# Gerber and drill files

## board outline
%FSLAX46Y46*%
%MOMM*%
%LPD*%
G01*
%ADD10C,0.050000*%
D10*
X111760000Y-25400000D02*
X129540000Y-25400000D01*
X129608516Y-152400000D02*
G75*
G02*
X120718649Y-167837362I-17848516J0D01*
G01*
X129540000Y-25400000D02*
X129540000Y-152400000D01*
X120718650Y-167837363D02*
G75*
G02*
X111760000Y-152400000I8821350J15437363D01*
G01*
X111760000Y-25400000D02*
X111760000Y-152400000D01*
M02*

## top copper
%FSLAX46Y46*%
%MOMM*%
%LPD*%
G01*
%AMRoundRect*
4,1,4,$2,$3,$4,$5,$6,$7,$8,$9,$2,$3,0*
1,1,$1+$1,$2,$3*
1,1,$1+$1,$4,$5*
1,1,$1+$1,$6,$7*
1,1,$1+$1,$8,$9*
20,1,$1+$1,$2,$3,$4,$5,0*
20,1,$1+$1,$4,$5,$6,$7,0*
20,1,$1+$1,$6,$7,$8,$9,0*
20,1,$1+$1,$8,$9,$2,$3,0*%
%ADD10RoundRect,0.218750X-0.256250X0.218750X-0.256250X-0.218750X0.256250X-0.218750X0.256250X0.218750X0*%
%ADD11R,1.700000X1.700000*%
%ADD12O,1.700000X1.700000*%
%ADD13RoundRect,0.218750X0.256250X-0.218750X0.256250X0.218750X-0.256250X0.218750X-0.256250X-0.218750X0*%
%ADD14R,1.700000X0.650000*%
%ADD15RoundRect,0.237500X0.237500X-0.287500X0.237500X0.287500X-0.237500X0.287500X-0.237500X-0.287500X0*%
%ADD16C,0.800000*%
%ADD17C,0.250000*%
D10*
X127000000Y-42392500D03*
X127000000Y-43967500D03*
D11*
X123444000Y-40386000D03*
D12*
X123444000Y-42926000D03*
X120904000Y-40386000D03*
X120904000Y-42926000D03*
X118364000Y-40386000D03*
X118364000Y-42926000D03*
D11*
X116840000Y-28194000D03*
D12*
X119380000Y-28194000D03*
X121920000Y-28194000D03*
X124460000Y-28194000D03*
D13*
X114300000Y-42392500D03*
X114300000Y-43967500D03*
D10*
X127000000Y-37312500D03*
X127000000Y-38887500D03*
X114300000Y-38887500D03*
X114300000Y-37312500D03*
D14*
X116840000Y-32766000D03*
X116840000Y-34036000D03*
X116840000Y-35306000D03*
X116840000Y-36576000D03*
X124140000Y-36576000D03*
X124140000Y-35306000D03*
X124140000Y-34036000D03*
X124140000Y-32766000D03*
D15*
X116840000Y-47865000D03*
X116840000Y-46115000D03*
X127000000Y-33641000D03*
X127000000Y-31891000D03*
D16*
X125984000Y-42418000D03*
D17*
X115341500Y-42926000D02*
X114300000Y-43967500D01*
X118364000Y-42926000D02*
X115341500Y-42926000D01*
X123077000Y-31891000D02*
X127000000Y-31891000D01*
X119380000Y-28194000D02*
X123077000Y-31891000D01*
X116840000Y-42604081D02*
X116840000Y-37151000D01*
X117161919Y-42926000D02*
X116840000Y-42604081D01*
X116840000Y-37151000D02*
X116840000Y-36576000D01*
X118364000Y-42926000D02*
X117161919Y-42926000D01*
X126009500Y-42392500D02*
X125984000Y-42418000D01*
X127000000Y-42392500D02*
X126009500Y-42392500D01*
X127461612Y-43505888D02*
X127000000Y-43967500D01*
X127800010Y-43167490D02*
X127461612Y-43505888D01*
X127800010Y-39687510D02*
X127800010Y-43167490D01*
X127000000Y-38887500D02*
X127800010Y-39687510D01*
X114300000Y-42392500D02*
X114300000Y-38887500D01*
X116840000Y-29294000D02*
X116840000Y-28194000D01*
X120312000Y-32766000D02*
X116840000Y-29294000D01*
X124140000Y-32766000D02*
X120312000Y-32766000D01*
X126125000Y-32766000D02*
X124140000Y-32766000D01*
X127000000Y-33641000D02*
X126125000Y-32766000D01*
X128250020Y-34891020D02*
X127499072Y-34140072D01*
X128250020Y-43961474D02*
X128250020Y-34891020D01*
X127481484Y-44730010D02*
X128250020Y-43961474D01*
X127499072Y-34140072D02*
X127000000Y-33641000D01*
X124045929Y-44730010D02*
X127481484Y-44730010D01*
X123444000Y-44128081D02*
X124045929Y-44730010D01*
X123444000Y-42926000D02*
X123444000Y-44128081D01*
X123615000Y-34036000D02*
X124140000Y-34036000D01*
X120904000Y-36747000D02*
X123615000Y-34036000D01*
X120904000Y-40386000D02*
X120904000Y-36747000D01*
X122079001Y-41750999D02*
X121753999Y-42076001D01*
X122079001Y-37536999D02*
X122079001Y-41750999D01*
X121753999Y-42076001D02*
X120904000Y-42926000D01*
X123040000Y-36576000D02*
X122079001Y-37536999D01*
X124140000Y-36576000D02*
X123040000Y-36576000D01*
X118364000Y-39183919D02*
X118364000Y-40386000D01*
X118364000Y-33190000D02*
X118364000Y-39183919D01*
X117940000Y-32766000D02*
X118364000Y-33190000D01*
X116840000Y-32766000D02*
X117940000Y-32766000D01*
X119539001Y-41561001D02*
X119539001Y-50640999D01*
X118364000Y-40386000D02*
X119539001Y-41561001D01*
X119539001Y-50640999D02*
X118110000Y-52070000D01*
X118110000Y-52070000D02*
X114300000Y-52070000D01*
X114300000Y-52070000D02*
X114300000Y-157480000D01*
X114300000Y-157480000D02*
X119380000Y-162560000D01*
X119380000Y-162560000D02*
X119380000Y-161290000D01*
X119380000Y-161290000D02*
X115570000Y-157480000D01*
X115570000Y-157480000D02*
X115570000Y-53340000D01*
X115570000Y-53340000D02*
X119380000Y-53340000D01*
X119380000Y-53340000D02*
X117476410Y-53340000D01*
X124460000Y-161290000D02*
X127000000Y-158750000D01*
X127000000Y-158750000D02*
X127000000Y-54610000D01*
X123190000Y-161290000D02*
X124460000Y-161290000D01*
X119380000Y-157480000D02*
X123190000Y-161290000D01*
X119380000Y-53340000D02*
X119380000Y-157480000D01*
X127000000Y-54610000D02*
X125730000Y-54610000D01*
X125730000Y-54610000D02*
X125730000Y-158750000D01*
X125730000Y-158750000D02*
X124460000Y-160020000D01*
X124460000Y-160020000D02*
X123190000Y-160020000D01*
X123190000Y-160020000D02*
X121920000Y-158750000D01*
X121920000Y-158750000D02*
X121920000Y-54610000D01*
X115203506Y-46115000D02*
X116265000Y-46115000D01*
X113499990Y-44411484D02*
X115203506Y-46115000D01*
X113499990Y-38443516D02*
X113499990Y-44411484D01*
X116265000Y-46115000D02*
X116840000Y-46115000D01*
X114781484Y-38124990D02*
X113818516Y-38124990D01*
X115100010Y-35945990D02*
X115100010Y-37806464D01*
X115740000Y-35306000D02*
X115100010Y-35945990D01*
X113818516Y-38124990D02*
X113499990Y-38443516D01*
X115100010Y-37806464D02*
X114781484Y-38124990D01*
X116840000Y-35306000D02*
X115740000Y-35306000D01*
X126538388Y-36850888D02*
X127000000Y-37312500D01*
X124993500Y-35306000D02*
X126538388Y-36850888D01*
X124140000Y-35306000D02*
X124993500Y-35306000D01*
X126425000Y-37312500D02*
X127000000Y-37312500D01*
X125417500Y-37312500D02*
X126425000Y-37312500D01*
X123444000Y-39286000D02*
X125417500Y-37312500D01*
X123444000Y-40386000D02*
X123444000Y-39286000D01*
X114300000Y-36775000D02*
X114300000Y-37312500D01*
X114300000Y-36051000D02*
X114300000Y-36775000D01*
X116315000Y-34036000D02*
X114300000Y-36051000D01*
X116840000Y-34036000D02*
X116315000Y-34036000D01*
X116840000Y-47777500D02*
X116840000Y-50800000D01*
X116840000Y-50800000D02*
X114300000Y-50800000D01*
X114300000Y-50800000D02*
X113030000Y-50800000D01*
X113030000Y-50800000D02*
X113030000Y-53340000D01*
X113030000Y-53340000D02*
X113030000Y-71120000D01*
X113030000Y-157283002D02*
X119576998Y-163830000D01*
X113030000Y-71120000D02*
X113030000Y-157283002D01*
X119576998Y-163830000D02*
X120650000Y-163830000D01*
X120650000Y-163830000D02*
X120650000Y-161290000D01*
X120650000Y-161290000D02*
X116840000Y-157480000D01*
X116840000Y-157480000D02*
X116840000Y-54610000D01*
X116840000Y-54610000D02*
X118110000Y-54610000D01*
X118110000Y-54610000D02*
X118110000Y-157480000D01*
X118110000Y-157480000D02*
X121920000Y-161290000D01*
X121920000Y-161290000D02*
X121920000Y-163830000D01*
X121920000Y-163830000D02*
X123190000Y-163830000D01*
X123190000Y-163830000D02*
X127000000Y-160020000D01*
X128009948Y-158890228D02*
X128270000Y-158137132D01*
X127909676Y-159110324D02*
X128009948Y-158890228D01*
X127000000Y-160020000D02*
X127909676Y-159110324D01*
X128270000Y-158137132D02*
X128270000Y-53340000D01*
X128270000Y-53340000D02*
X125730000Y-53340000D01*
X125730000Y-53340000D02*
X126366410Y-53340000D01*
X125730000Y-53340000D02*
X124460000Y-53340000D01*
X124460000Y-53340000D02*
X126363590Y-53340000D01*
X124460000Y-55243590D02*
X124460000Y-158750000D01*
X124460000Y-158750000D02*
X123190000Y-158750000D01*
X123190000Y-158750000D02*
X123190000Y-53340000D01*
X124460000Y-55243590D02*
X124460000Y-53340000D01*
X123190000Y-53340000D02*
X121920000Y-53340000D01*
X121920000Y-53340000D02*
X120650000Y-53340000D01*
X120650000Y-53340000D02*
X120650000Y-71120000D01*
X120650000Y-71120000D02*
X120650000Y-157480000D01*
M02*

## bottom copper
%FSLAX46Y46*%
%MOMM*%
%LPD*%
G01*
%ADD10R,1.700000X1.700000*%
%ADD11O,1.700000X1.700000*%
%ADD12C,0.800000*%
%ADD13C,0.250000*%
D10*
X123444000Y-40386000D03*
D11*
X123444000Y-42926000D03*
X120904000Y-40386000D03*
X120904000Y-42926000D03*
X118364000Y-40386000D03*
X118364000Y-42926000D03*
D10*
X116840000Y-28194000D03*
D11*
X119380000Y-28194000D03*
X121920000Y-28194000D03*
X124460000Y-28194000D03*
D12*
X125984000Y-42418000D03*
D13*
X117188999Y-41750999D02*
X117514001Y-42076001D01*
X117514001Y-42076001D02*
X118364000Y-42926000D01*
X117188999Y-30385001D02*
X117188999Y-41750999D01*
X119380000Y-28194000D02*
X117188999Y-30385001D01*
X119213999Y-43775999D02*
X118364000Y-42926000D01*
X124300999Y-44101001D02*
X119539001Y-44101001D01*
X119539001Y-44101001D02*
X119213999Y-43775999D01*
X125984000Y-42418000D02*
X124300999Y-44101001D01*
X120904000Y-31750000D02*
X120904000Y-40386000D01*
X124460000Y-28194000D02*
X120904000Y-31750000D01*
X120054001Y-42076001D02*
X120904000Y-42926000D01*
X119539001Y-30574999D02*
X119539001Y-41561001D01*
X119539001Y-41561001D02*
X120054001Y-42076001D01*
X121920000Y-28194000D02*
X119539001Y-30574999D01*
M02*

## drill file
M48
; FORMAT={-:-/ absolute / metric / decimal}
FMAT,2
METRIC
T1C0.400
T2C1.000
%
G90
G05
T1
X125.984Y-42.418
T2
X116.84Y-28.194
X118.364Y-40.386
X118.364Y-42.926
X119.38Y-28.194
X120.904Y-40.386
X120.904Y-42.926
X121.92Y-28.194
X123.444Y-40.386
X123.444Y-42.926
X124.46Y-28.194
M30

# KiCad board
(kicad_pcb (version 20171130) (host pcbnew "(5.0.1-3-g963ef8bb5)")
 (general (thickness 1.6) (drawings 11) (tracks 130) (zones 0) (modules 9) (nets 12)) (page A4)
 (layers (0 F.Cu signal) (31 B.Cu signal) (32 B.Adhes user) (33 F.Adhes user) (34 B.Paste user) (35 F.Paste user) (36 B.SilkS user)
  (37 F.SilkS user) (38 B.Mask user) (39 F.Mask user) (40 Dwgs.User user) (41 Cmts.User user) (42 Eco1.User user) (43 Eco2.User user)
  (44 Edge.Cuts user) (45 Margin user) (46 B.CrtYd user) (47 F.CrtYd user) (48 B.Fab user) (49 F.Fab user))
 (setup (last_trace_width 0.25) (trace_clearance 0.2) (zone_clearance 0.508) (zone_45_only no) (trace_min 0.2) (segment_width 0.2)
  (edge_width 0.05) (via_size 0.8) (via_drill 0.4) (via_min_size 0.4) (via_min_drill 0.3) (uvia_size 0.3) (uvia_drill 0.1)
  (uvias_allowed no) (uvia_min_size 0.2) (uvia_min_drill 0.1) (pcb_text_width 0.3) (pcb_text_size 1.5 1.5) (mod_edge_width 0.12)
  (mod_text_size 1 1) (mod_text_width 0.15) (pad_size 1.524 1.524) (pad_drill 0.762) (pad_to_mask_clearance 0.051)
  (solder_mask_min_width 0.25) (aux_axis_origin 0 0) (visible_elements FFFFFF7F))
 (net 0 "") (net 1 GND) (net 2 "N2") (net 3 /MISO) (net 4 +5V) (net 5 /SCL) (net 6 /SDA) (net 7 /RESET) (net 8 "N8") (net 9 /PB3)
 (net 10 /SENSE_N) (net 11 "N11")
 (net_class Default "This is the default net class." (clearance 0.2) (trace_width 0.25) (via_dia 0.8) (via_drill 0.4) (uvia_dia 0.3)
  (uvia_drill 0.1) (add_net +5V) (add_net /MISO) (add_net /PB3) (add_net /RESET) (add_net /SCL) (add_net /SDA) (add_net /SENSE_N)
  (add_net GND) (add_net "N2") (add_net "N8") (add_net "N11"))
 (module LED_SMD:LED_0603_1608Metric (layer F.Cu) (at 127 43.18 270)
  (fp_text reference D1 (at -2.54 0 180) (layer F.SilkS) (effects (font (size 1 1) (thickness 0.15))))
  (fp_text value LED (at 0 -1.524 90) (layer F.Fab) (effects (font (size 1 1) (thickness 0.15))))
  (pad 1 smd roundrect (at -0.7875 0 270) (size 0.875 0.95) (layers F.Cu F.Paste F.Mask) (roundrect_rratio 0.25) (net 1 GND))
  (pad 2 smd roundrect (at 0.7875 0 270) (size 0.875 0.95) (layers F.Cu F.Paste F.Mask) (roundrect_rratio 0.25) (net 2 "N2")))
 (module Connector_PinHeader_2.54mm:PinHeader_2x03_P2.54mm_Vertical (layer F.Cu) (at 123.444 40.386 270)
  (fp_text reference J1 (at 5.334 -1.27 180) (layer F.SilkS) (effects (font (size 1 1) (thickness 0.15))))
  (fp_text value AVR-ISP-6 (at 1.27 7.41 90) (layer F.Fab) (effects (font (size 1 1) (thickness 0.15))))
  (pad 1 thru_hole rect (at 0 0 270) (size 1.7 1.7) (drill 1) (layers *.Cu *.Mask) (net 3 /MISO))
  (pad 2 thru_hole oval (at 2.54 0 270) (size 1.7 1.7) (drill 1) (layers *.Cu *.Mask) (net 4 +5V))
  (pad 3 thru_hole oval (at 0 2.54 270) (size 1.7 1.7) (drill 1) (layers *.Cu *.Mask) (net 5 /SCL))
  (pad 4 thru_hole oval (at 2.54 2.54 270) (size 1.7 1.7) (drill 1) (layers *.Cu *.Mask) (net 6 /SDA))
  (pad 5 thru_hole oval (at 0 5.08 270) (size 1.7 1.7) (drill 1) (layers *.Cu *.Mask) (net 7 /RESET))
  (pad 6 thru_hole oval (at 2.54 5.08 270) (size 1.7 1.7) (drill 1) (layers *.Cu *.Mask) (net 1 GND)))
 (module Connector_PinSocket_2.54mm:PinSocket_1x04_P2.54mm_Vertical (layer F.Cu) (at 116.84 28.194 90)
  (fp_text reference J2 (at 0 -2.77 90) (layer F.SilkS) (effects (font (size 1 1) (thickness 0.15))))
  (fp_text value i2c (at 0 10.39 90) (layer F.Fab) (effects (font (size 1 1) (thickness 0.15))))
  (pad 1 thru_hole rect (at 0 0 90) (size 1.7 1.7) (drill 1) (layers *.Cu *.Mask) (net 4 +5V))
  (pad 2 thru_hole oval (at 0 2.54 90) (size 1.7 1.7) (drill 1) (layers *.Cu *.Mask) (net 1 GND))
  (pad 3 thru_hole oval (at 0 5.08 90) (size 1.7 1.7) (drill 1) (layers *.Cu *.Mask) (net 6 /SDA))
  (pad 4 thru_hole oval (at 0 7.62 90) (size 1.7 1.7) (drill 1) (layers *.Cu *.Mask) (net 5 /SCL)))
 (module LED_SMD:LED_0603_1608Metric (layer F.Cu) (at 114.3 43.18 90)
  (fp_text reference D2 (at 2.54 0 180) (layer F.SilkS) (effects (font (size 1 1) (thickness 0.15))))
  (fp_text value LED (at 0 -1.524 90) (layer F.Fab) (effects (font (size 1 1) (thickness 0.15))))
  (pad 2 smd roundrect (at 0.7875 0 90) (size 0.875 0.95) (layers F.Cu F.Paste F.Mask) (roundrect_rratio 0.25) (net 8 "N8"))
  (pad 1 smd roundrect (at -0.7875 0 90) (size 0.875 0.95) (layers F.Cu F.Paste F.Mask) (roundrect_rratio 0.25) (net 1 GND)))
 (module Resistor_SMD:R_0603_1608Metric (layer F.Cu) (at 127 38.1 270)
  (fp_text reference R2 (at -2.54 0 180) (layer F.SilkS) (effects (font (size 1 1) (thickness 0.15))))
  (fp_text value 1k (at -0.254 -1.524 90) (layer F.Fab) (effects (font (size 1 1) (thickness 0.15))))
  (pad 1 smd roundrect (at -0.7875 0 270) (size 0.875 0.95) (layers F.Cu F.Paste F.Mask) (roundrect_rratio 0.25) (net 3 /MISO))
  (pad 2 smd roundrect (at 0.7875 0 270) (size 0.875 0.95) (layers F.Cu F.Paste F.Mask) (roundrect_rratio 0.25) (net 2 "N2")))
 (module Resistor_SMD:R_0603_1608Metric (layer F.Cu) (at 114.3 38.1 270)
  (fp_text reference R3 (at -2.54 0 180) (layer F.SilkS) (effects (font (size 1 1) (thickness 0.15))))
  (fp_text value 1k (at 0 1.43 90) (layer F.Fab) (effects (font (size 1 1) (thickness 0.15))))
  (pad 2 smd roundrect (at 0.7875 0 270) (size 0.875 0.95) (layers F.Cu F.Paste F.Mask) (roundrect_rratio 0.25) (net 8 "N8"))
  (pad 1 smd roundrect (at -0.7875 0 270) (size 0.875 0.95) (layers F.Cu F.Paste F.Mask) (roundrect_rratio 0.25) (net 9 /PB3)))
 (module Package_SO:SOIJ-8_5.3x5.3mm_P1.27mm (layer F.Cu) (at 120.49 34.671)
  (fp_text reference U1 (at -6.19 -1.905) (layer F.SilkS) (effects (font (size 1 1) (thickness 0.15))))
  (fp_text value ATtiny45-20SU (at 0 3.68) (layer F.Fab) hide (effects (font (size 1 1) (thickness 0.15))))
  (pad 1 smd rect (at -3.65 -1.905) (size 1.7 0.65) (layers F.Cu F.Paste F.Mask) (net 7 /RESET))
  (pad 2 smd rect (at -3.65 -0.635) (size 1.7 0.65) (layers F.Cu F.Paste F.Mask) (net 9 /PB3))
  (pad 3 smd rect (at -3.65 0.635) (size 1.7 0.65) (layers F.Cu F.Paste F.Mask) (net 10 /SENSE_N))
  (pad 4 smd rect (at -3.65 1.905) (size 1.7 0.65) (layers F.Cu F.Paste F.Mask) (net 1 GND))
  (pad 5 smd rect (at 3.65 1.905) (size 1.7 0.65) (layers F.Cu F.Paste F.Mask) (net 6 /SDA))
  (pad 6 smd rect (at 3.65 0.635) (size 1.7 0.65) (layers F.Cu F.Paste F.Mask) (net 3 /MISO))
  (pad 7 smd rect (at 3.65 -0.635) (size 1.7 0.65) (layers F.Cu F.Paste F.Mask) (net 5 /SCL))
  (pad 8 smd rect (at 3.65 -1.905) (size 1.7 0.65) (layers F.Cu F.Paste F.Mask) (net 4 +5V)))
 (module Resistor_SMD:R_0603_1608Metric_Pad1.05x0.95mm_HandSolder (layer F.Cu) (at 116.84 46.99 90)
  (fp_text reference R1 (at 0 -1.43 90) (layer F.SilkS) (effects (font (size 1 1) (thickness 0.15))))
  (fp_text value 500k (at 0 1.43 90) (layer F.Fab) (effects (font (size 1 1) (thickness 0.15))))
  (pad 1 smd roundrect (at -0.875 0 90) (size 1.05 0.95) (layers F.Cu F.Paste F.Mask) (roundrect_rratio 0.25) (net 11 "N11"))
  (pad 2 smd roundrect (at 0.875 0 90) (size 1.05 0.95) (layers F.Cu F.Paste F.Mask) (roundrect_rratio 0.25) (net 10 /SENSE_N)))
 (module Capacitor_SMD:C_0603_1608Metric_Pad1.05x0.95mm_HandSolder (layer F.Cu) (at 127 32.766 90)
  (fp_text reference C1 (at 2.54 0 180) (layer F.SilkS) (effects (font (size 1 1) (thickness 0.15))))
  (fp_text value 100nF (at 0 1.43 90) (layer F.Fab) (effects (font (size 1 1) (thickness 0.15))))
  (pad 1 smd roundrect (at -0.875 0 90) (size 1.05 0.95) (layers F.Cu F.Paste F.Mask) (roundrect_rratio 0.25) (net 4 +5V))
  (pad 2 smd roundrect (at 0.875 0 90) (size 1.05 0.95) (layers F.Cu F.Paste F.Mask) (roundrect_rratio 0.25) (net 1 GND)))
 (gr_line (start 111.76 25.4) (end 129.54 25.4) (layer Edge.Cuts) (width 0.05))
 (gr_arc (start 111.76 152.4) (end 120.718649 167.837362) (angle -59.87243964) (layer Edge.Cuts) (width 0.05))
 (gr_line (start 129.54 25.4) (end 129.54 152.4) (layer Edge.Cuts) (width 0.05))
 (gr_arc (start 129.54 152.4) (end 111.76 152.4) (angle -60.2551187) (layer Edge.Cuts) (width 0.05))
 (gr_line (start 111.76 25.4) (end 111.76 152.4) (layer Edge.Cuts) (width 0.05))
 (segment (start 115.3415 42.926) (end 114.3 43.9675) (width 0.25) (layer F.Cu) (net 1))
 (segment (start 118.364 42.926) (end 115.3415 42.926) (width 0.25) (layer F.Cu) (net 1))
 (segment (start 123.077 31.891) (end 127 31.891) (width 0.25) (layer F.Cu) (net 1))
 (segment (start 119.38 28.194) (end 123.077 31.891) (width 0.25) (layer F.Cu) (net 1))
 (segment (start 116.84 42.604081) (end 116.84 37.151) (width 0.25) (layer F.Cu) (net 1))
 (segment (start 117.161919 42.926) (end 116.84 42.604081) (width 0.25) (layer F.Cu) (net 1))
 (segment (start 116.84 37.151) (end 116.84 36.576) (width 0.25) (layer F.Cu) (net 1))
 (segment (start 118.364 42.926) (end 117.161919 42.926) (width 0.25) (layer F.Cu) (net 1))
 (segment (start 117.188999 41.750999) (end 117.514001 42.076001) (width 0.25) (layer B.Cu) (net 1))
 (segment (start 117.514001 42.076001) (end 118.364 42.926) (width 0.25) (layer B.Cu) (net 1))
 (segment (start 117.188999 30.385001) (end 117.188999 41.750999) (width 0.25) (layer B.Cu) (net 1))
 (segment (start 119.38 28.194) (end 117.188999 30.385001) (width 0.25) (layer B.Cu) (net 1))
 (via (at 125.984 42.418) (size 0.8) (drill 0.4) (layers F.Cu B.Cu) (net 1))
 (segment (start 126.0095 42.3925) (end 125.984 42.418) (width 0.25) (layer F.Cu) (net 1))
 (segment (start 127 42.3925) (end 126.0095 42.3925) (width 0.25) (layer F.Cu) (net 1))
 (segment (start 119.213999 43.775999) (end 118.364 42.926) (width 0.25) (layer B.Cu) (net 1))
 (segment (start 124.300999 44.101001) (end 119.539001 44.101001) (width 0.25) (layer B.Cu) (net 1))
 (segment (start 119.539001 44.101001) (end 119.213999 43.775999) (width 0.25) (layer B.Cu) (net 1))
 (segment (start 125.984 42.418) (end 124.300999 44.101001) (width 0.25) (layer B.Cu) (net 1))
 (segment (start 127.461612 43.505888) (end 127 43.9675) (width 0.25) (layer F.Cu) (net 2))
 (segment (start 127.80001 43.16749) (end 127.461612 43.505888) (width 0.25) (layer F.Cu) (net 2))
 (segment (start 127.80001 39.68751) (end 127.80001 43.16749) (width 0.25) (layer F.Cu) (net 2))
 (segment (start 127 38.8875) (end 127.80001 39.68751) (width 0.25) (layer F.Cu) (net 2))
 (segment (start 114.3 42.3925) (end 114.3 38.8875) (width 0.25) (layer F.Cu) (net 8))
 (segment (start 116.84 29.294) (end 116.84 28.194) (width 0.25) (layer F.Cu) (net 4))
 (segment (start 120.312 32.766) (end 116.84 29.294) (width 0.25) (layer F.Cu) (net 4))
 (segment (start 124.14 32.766) (end 120.312 32.766) (width 0.25) (layer F.Cu) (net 4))
 (segment (start 126.125 32.766) (end 124.14 32.766) (width 0.25) (layer F.Cu) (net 4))
 (segment (start 127 33.641) (end 126.125 32.766) (width 0.25) (layer F.Cu) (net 4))
 (segment (start 128.25002 34.89102) (end 127.499072 34.140072) (width 0.25) (layer F.Cu) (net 4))
 (segment (start 128.25002 43.961474) (end 128.25002 34.89102) (width 0.25) (layer F.Cu) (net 4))
 (segment (start 127.481484 44.73001) (end 128.25002 43.961474) (width 0.25) (layer F.Cu) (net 4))
 (segment (start 127.499072 34.140072) (end 127 33.641) (width 0.25) (layer F.Cu) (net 4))
 (segment (start 124.045929 44.73001) (end 127.481484 44.73001) (width 0.25) (layer F.Cu) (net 4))
 (segment (start 123.444 44.128081) (end 124.045929 44.73001) (width 0.25) (layer F.Cu) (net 4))
 (segment (start 123.444 42.926) (end 123.444 44.128081) (width 0.25) (layer F.Cu) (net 4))
 (segment (start 123.615 34.036) (end 124.14 34.036) (width 0.25) (layer F.Cu) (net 5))
 (segment (start 120.904 36.747) (end 123.615 34.036) (width 0.25) (layer F.Cu) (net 5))
 (segment (start 120.904 40.386) (end 120.904 36.747) (width 0.25) (layer F.Cu) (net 5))
 (segment (start 120.904 31.75) (end 120.904 40.386) (width 0.25) (layer B.Cu) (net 5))
 (segment (start 124.46 28.194) (end 120.904 31.75) (width 0.25) (layer B.Cu) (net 5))
 (segment (start 120.054001 42.076001) (end 120.904 42.926) (width 0.25) (layer B.Cu) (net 6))
 (segment (start 119.539001 30.574999) (end 119.539001 41.561001) (width 0.25) (layer B.Cu) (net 6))
 (segment (start 119.539001 41.561001) (end 120.054001 42.076001) (width 0.25) (layer B.Cu) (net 6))
 (segment (start 121.92 28.194) (end 119.539001 30.574999) (width 0.25) (layer B.Cu) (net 6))
 (segment (start 122.079001 41.750999) (end 121.753999 42.076001) (width 0.25) (layer F.Cu) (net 6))
 (segment (start 122.079001 37.536999) (end 122.079001 41.750999) (width 0.25) (layer F.Cu) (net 6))
 (segment (start 121.753999 42.076001) (end 120.904 42.926) (width 0.25) (layer F.Cu) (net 6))
 (segment (start 123.04 36.576) (end 122.079001 37.536999) (width 0.25) (layer F.Cu) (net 6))
 (segment (start 124.14 36.576) (end 123.04 36.576) (width 0.25) (layer F.Cu) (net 6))
 (segment (start 118.364 39.183919) (end 118.364 40.386) (width 0.25) (layer F.Cu) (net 7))
 (segment (start 118.364 33.19) (end 118.364 39.183919) (width 0.25) (layer F.Cu) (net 7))
 (segment (start 117.94 32.766) (end 118.364 33.19) (width 0.25) (layer F.Cu) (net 7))
 (segment (start 116.84 32.766) (end 117.94 32.766) (width 0.25) (layer F.Cu) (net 7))
 (segment (start 119.539001 41.561001) (end 119.539001 50.640999) (width 0.25) (layer F.Cu) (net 7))
 (segment (start 118.364 40.386) (end 119.539001 41.561001) (width 0.25) (layer F.Cu) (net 7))
 (segment (start 119.539001 50.640999) (end 118.11 52.07) (width 0.25) (layer F.Cu) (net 7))
 (segment (start 118.11 52.07) (end 114.3 52.07) (width 0.25) (layer F.Cu) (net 7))
 (segment (start 114.3 52.07) (end 114.3 157.48) (width 0.25) (layer F.Cu) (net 7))
 (segment (start 114.3 157.48) (end 119.38 162.56) (width 0.25) (layer F.Cu) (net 7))
 (segment (start 119.38 162.56) (end 119.38 161.29) (width 0.25) (layer F.Cu) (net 7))
 (segment (start 119.38 161.29) (end 115.57 157.48) (width 0.25) (layer F.Cu) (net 7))
 (segment (start 115.57 157.48) (end 115.57 53.34) (width 0.25) (layer F.Cu) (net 7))
 (segment (start 115.57 53.34) (end 119.38 53.34) (width 0.25) (layer F.Cu) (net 7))
 (segment (start 119.38 53.34) (end 117.47641 53.34) (width 0.25) (layer F.Cu) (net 7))
 (segment (start 124.46 161.29) (end 127 158.75) (width 0.25) (layer F.Cu) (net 7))
 (segment (start 127 158.75) (end 127 54.61) (width 0.25) (layer F.Cu) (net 7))
 (segment (start 123.19 161.29) (end 124.46 161.29) (width 0.25) (layer F.Cu) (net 7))
 (segment (start 119.38 157.48) (end 123.19 161.29) (width 0.25) (layer F.Cu) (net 7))
 (segment (start 119.38 53.34) (end 119.38 157.48) (width 0.25) (layer F.Cu) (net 7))
 (segment (start 127 54.61) (end 125.73 54.61) (width 0.25) (layer F.Cu) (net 7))
 (segment (start 125.73 54.61) (end 125.73 158.75) (width 0.25) (layer F.Cu) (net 7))
 (segment (start 125.73 158.75) (end 124.46 160.02) (width 0.25) (layer F.Cu) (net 7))
 (segment (start 124.46 160.02) (end 123.19 160.02) (width 0.25) (layer F.Cu) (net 7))
 (segment (start 123.19 160.02) (end 121.92 158.75) (width 0.25) (layer F.Cu) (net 7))
 (segment (start 121.92 158.75) (end 121.92 54.61) (width 0.25) (layer F.Cu) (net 7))
 (segment (start 115.203506 46.115) (end 116.265 46.115) (width 0.25) (layer F.Cu) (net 10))
 (segment (start 113.49999 44.411484) (end 115.203506 46.115) (width 0.25) (layer F.Cu) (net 10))
 (segment (start 113.49999 38.443516) (end 113.49999 44.411484) (width 0.25) (layer F.Cu) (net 10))
 (segment (start 116.265 46.115) (end 116.84 46.115) (width 0.25) (layer F.Cu) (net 10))
 (segment (start 114.781484 38.12499) (end 113.818516 38.12499) (width 0.25) (layer F.Cu) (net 10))
 (segment (start 115.10001 35.94599) (end 115.10001 37.806464) (width 0.25) (layer F.Cu) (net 10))
 (segment (start 115.74 35.306) (end 115.10001 35.94599) (width 0.25) (layer F.Cu) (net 10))
 (segment (start 113.818516 38.12499) (end 113.49999 38.443516) (width 0.25) (layer F.Cu) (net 10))
 (segment (start 115.10001 37.806464) (end 114.781484 38.12499) (width 0.25) (layer F.Cu) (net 10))
 (segment (start 116.84 35.306) (end 115.74 35.306) (width 0.25) (layer F.Cu) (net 10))
 (segment (start 126.538388 36.850888) (end 127 37.3125) (width 0.25) (layer F.Cu) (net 3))
 (segment (start 124.9935 35.306) (end 126.538388 36.850888) (width 0.25) (layer F.Cu) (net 3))
 (segment (start 124.14 35.306) (end 124.9935 35.306) (width 0.25) (layer F.Cu) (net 3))
 (segment (start 126.425 37.3125) (end 127 37.3125) (width 0.25) (layer F.Cu) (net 3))
 (segment (start 125.4175 37.3125) (end 126.425 37.3125) (width 0.25) (layer F.Cu) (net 3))
 (segment (start 123.444 39.286) (end 125.4175 37.3125) (width 0.25) (layer F.Cu) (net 3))
 (segment (start 123.444 40.386) (end 123.444 39.286) (width 0.25) (layer F.Cu) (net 3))
 (segment (start 114.3 36.775) (end 114.3 37.3125) (width 0.25) (layer F.Cu) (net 9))
 (segment (start 114.3 36.051) (end 114.3 36.775) (width 0.25) (layer F.Cu) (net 9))
 (segment (start 116.315 34.036) (end 114.3 36.051) (width 0.25) (layer F.Cu) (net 9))
 (segment (start 116.84 34.036) (end 116.315 34.036) (width 0.25) (layer F.Cu) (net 9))
 (segment (start 116.84 47.7775) (end 116.84 50.8) (width 0.25) (layer F.Cu) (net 11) (status 10))
 (segment (start 116.84 50.8) (end 114.3 50.8) (width 0.25) (layer F.Cu) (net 11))
 (segment (start 114.3 50.8) (end 113.03 50.8) (width 0.25) (layer F.Cu) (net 11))
 (segment (start 113.03 50.8) (end 113.03 53.34) (width 0.25) (layer F.Cu) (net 11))
 (segment (start 113.03 53.34) (end 113.03 71.12) (width 0.25) (layer F.Cu) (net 11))
 (segment (start 113.03 157.283002) (end 119.576998 163.83) (width 0.25) (layer F.Cu) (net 11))
 (segment (start 113.03 71.12) (end 113.03 157.283002) (width 0.25) (layer F.Cu) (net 11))
 (segment (start 119.576998 163.83) (end 120.65 163.83) (width 0.25) (layer F.Cu) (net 11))
 (segment (start 120.65 163.83) (end 120.65 161.29) (width 0.25) (layer F.Cu) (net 11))
 (segment (start 120.65 161.29) (end 116.84 157.48) (width 0.25) (layer F.Cu) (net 11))
 (segment (start 116.84 157.48) (end 116.84 54.61) (width 0.25) (layer F.Cu) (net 11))
 (segment (start 116.84 54.61) (end 118.11 54.61) (width 0.25) (layer F.Cu) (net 11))
 (segment (start 118.11 54.61) (end 118.11 157.48) (width 0.25) (layer F.Cu) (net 11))
 (segment (start 118.11 157.48) (end 121.92 161.29) (width 0.25) (layer F.Cu) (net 11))
 (segment (start 121.92 161.29) (end 121.92 163.83) (width 0.25) (layer F.Cu) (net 11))
 (segment (start 121.92 163.83) (end 123.19 163.83) (width 0.25) (layer F.Cu) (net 11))
 (segment (start 123.19 163.83) (end 127 160.02) (width 0.25) (layer F.Cu) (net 11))
 (segment (start 128.009948 158.890228) (end 128.27 158.137132) (width 0.25) (layer F.Cu) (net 11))
 (segment (start 127.909676 159.110324) (end 128.009948 158.890228) (width 0.25) (layer F.Cu) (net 11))
 (segment (start 127 160.02) (end 127.909676 159.110324) (width 0.25) (layer F.Cu) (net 11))
 (segment (start 128.27 158.137132) (end 128.27 53.34) (width 0.25) (layer F.Cu) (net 11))
 (segment (start 128.27 53.34) (end 125.73 53.34) (width 0.25) (layer F.Cu) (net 11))
 (segment (start 125.73 53.34) (end 126.36641 53.34) (width 0.25) (layer F.Cu) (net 11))
 (segment (start 125.73 53.34) (end 124.46 53.34) (width 0.25) (layer F.Cu) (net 11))
 (segment (start 124.46 53.34) (end 126.36359 53.34) (width 0.25) (layer F.Cu) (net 11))
 (segment (start 124.46 55.24359) (end 124.46 158.75) (width 0.25) (layer F.Cu) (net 11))
 (segment (start 124.46 158.75) (end 123.19 158.75) (width 0.25) (layer F.Cu) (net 11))
 (segment (start 123.19 158.75) (end 123.19 53.34) (width 0.25) (layer F.Cu) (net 11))
 (segment (start 124.46 55.24359) (end 124.46 53.34) (width 0.25) (layer F.Cu) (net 11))
 (segment (start 123.19 53.34) (end 121.92 53.34) (width 0.25) (layer F.Cu) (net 11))
 (segment (start 121.92 53.34) (end 120.65 53.34) (width 0.25) (layer F.Cu) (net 11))
 (segment (start 120.65 53.34) (end 120.65 71.12) (width 0.25) (layer F.Cu) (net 11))
 (segment (start 120.65 71.12) (end 120.65 157.48) (width 0.25) (layer F.Cu) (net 11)))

